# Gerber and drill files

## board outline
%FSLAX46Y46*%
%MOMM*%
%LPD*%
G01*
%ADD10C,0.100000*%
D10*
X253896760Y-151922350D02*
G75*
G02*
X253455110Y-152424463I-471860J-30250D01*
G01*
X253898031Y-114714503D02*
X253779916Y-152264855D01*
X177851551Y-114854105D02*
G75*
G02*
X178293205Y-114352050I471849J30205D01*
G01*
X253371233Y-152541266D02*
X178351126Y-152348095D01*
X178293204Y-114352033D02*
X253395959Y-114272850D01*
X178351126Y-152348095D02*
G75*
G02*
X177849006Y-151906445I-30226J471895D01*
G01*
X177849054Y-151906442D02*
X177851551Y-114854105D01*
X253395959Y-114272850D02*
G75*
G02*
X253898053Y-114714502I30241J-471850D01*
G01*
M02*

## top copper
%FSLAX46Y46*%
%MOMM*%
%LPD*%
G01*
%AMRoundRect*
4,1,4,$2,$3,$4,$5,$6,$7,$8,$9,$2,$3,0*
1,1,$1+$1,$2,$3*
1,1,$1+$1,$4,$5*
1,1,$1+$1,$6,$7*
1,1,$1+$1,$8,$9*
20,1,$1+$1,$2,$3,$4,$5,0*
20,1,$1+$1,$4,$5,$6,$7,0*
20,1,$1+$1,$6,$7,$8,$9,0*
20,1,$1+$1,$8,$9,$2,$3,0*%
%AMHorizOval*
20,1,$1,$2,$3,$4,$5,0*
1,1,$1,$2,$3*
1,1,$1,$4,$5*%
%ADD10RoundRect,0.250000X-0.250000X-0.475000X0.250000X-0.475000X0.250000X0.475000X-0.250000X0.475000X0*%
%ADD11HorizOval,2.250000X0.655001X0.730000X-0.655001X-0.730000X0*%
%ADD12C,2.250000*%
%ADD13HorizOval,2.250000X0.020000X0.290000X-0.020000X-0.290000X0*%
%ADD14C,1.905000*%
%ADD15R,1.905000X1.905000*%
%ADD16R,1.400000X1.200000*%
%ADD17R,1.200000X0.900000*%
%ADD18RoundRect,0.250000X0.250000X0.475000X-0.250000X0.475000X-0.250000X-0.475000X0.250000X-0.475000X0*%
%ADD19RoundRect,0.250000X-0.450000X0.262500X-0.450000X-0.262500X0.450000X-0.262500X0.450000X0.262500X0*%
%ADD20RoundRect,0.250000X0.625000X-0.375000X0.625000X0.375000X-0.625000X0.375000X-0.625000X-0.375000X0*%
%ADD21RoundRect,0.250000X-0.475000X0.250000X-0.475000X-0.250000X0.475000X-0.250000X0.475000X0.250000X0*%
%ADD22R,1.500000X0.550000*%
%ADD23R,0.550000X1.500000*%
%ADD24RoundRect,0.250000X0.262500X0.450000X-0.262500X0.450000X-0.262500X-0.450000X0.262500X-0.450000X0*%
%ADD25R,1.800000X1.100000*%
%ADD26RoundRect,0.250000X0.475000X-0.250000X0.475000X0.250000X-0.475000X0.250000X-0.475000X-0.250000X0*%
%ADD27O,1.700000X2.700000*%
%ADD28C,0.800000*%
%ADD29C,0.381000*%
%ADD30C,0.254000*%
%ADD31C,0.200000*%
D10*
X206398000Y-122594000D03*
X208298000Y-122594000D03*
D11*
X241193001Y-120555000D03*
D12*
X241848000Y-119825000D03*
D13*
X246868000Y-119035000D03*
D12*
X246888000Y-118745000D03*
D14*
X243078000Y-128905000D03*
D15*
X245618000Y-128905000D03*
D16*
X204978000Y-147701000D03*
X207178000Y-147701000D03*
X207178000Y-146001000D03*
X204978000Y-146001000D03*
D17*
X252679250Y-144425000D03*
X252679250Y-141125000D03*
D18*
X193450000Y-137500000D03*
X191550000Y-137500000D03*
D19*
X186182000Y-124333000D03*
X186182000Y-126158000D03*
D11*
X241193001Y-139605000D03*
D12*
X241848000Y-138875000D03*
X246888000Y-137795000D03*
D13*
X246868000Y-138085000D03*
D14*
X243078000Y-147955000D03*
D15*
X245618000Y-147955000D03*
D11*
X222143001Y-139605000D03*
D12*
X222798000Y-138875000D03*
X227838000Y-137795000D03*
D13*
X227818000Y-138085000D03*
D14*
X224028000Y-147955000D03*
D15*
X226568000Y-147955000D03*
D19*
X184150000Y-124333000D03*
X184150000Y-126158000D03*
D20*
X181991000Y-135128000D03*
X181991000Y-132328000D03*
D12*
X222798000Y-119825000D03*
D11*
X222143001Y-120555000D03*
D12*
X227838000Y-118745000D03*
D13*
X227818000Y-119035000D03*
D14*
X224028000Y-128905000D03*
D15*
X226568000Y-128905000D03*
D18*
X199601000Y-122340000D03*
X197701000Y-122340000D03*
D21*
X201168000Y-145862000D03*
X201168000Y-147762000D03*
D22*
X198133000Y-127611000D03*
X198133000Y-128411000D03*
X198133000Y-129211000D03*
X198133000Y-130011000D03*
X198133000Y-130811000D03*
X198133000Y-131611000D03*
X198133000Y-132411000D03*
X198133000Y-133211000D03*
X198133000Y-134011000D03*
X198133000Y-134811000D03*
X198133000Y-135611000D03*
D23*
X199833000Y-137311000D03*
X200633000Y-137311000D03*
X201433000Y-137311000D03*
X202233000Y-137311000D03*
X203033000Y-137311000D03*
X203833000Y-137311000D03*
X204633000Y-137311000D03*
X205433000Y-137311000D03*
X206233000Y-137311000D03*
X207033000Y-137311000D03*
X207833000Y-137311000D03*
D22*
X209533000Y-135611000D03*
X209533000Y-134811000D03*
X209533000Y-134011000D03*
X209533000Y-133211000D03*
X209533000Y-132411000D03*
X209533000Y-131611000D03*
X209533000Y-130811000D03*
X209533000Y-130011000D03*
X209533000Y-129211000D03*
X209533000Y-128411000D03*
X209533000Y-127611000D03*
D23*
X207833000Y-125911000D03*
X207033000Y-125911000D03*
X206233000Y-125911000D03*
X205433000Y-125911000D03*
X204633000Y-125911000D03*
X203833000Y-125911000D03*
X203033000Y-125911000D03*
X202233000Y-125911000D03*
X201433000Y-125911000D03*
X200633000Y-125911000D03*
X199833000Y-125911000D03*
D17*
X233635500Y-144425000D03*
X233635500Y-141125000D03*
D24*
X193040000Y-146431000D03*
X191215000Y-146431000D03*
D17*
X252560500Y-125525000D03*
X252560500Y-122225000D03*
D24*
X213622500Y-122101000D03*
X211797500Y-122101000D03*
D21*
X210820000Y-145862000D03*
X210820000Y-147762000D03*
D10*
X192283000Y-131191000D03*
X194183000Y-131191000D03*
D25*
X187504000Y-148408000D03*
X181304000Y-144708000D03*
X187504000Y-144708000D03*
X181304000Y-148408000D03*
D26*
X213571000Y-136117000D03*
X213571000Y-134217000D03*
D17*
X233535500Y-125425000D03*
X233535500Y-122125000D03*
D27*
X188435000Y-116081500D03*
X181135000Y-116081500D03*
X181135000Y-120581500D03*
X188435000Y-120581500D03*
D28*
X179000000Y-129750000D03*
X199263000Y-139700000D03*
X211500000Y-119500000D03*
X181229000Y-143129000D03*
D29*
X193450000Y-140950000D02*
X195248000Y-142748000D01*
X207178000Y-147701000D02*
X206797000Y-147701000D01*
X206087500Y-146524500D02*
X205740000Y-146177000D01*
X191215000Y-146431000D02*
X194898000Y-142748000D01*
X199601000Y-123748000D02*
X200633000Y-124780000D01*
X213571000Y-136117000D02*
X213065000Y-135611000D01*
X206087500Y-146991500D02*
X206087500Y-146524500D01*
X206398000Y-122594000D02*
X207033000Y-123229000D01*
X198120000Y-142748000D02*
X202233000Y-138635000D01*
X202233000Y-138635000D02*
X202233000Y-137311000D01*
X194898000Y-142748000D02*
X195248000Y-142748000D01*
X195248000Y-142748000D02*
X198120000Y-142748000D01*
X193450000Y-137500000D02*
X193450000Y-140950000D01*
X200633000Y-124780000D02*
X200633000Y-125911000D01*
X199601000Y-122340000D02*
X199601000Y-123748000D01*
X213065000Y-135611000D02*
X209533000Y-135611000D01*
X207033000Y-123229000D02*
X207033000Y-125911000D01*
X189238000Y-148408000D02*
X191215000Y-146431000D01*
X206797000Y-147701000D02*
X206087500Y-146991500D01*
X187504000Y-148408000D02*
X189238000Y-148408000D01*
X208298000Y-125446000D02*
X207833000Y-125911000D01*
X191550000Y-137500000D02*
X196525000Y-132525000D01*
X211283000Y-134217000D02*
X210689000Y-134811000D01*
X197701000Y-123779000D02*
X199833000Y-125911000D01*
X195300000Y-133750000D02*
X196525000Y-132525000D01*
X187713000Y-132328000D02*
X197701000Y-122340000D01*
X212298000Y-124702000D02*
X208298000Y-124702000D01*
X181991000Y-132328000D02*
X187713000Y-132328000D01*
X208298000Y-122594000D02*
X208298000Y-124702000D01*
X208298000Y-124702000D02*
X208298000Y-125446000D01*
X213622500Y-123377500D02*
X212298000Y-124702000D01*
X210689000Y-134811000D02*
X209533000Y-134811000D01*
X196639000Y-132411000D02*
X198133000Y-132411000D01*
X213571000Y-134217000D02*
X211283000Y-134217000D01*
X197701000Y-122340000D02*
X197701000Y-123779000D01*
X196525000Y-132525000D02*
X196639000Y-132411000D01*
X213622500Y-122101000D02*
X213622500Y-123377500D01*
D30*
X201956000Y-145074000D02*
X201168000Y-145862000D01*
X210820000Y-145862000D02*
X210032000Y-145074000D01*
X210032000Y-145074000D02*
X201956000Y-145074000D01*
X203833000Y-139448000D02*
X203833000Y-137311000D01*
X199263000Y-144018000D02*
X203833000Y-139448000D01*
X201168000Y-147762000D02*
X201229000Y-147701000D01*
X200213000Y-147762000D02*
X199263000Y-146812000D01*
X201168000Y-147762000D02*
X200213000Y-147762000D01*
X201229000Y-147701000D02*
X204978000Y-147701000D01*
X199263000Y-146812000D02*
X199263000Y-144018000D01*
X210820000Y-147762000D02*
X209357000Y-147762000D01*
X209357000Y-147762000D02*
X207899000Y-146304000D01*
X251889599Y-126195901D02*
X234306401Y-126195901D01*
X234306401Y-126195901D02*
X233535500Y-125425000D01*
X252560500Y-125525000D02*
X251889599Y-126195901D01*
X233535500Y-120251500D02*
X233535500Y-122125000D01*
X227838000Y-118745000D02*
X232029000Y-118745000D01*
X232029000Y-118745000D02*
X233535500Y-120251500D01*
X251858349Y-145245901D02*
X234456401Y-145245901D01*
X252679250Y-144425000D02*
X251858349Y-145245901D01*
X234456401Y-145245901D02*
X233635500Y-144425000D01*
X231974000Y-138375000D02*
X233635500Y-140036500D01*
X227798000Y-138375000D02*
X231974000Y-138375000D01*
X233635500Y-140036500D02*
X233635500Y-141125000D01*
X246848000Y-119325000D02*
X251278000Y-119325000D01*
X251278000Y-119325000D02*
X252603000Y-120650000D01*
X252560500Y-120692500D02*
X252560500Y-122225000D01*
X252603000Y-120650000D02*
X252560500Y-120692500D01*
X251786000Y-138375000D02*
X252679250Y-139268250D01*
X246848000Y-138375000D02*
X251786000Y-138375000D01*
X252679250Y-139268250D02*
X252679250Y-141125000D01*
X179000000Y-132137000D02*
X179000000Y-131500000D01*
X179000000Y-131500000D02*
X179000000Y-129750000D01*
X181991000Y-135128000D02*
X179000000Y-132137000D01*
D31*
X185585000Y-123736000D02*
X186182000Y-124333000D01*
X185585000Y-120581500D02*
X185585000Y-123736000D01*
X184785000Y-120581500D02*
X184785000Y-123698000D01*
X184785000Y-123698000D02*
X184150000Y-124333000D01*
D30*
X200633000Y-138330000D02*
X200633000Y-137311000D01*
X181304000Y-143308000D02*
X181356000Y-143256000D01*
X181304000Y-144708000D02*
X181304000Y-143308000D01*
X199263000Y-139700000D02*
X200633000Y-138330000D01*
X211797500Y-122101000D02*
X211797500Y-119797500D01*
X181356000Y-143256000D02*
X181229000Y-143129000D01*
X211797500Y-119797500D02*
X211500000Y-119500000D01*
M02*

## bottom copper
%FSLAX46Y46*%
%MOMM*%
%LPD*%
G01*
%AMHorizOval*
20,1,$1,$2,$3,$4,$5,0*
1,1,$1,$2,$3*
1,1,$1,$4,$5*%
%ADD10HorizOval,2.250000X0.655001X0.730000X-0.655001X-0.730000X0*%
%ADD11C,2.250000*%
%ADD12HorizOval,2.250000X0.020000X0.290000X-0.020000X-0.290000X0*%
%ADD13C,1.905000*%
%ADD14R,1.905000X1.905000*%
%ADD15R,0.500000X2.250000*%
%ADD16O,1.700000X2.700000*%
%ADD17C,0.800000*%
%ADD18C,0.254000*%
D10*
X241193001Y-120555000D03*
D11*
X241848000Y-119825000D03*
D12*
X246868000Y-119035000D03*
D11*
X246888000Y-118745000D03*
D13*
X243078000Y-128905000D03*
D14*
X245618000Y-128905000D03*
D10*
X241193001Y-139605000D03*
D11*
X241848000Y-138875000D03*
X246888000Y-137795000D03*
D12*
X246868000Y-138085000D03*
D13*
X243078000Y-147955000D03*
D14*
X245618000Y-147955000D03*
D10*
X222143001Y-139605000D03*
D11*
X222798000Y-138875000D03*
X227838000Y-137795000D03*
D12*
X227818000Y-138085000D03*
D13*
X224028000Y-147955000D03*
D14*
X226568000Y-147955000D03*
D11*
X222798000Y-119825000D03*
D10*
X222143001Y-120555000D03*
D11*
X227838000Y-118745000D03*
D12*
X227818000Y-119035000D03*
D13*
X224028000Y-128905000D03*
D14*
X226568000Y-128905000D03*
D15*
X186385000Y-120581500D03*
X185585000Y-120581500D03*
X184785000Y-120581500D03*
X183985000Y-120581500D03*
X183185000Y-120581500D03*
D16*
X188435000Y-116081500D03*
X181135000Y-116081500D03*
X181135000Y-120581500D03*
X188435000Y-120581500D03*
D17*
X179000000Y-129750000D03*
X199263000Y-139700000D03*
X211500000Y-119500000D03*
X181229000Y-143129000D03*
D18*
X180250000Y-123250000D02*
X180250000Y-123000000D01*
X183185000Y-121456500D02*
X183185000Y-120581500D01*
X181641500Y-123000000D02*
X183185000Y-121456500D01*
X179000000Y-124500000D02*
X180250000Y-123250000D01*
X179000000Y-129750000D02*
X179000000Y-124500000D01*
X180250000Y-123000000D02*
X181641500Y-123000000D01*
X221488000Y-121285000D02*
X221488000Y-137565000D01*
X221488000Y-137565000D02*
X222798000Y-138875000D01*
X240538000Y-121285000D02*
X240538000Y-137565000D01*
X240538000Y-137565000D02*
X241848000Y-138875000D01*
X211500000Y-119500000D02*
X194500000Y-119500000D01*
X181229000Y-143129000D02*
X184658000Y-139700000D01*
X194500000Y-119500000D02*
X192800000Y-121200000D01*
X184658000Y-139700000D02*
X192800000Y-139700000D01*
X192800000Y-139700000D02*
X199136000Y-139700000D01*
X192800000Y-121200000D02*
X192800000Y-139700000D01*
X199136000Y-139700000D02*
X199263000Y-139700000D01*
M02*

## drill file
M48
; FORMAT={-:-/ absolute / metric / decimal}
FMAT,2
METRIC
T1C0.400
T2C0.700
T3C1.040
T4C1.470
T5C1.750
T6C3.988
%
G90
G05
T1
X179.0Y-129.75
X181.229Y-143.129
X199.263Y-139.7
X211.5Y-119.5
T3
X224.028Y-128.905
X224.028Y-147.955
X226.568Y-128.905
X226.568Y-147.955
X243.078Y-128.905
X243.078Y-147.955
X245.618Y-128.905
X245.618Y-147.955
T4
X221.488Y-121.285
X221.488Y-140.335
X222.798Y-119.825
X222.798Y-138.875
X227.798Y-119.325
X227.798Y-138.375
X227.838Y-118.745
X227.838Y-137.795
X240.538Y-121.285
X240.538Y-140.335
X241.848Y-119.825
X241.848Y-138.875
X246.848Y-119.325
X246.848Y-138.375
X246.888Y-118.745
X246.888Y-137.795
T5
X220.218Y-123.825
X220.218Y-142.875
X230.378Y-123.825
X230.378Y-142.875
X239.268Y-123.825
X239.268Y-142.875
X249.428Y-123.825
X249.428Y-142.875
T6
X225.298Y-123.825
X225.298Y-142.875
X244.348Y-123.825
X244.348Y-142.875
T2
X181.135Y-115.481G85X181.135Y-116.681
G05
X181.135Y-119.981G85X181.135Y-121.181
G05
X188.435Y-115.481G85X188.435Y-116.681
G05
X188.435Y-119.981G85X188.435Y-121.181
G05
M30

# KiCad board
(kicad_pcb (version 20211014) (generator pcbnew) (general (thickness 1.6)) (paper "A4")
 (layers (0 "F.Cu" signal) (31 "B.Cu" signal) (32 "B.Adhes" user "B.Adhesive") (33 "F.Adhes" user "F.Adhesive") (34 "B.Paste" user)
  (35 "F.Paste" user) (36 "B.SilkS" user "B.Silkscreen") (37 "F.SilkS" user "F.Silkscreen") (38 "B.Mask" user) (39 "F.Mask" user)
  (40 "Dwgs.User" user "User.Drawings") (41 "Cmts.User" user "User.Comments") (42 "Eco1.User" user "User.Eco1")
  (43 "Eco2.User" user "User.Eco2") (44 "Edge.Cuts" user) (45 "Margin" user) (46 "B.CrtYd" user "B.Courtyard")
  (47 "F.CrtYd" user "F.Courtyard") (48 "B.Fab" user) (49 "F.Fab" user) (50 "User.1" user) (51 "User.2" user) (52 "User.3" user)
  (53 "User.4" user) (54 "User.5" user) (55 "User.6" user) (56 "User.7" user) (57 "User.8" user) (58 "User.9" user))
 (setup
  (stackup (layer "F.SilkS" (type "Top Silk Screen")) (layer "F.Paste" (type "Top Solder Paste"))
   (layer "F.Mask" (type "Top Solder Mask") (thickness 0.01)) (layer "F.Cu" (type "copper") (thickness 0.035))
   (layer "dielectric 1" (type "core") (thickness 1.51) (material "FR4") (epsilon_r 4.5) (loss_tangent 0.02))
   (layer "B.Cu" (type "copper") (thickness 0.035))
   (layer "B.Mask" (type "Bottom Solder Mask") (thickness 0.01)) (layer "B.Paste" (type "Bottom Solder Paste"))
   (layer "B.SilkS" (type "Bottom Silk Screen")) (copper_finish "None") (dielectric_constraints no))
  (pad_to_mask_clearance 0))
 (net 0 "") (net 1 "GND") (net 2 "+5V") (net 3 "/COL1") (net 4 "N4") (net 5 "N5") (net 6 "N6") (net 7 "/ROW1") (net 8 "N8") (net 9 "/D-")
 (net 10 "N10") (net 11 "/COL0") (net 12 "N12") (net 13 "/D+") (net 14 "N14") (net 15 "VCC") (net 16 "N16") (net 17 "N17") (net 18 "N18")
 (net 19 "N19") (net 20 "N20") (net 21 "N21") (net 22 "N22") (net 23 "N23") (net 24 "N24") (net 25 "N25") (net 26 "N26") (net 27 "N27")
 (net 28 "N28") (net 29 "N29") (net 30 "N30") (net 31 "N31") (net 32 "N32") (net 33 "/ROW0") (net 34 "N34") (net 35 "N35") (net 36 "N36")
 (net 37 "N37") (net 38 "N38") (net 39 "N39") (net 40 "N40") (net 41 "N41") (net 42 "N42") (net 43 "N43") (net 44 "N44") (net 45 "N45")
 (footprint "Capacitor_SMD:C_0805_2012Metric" (layer "F.Cu") (at 207.348 122.594)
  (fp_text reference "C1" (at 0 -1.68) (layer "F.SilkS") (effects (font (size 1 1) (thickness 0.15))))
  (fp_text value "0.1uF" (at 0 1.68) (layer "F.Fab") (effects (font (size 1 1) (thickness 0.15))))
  (pad "1" smd roundrect (at -0.95 0) (size 1 1.45) (layers "F.Cu" "F.Paste" "F.Mask") (roundrect_rratio 0.25) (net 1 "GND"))
  (pad "2" smd roundrect (at 0.95 0) (size 1 1.45) (layers "F.Cu" "F.Paste" "F.Mask") (roundrect_rratio 0.25) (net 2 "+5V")))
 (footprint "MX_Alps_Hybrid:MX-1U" (layer "F.Cu") (at 244.348 123.825)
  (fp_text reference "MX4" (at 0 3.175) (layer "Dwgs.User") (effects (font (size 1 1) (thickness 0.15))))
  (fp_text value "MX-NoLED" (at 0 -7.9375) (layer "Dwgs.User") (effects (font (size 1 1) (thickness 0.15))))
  (pad "" np_thru_hole circle locked (at 0 0) (size 3.9878 3.9878) (drill 3.9878) (layers *.Cu *.Mask))
  (pad "" np_thru_hole circle locked (at 5.08 0 48.0996) (size 1.75 1.75) (drill 1.75) (layers *.Cu *.Mask))
  (pad "" np_thru_hole circle locked (at -5.08 0 48.0996) (size 1.75 1.75) (drill 1.75) (layers *.Cu *.Mask))
  (pad "1" thru_hole oval locked (at -3.81 -2.54 48.0996) (size 4.211556 2.25) (drill 1.47 (offset 0.980778 0)) (layers *.Cu "B.Mask")
   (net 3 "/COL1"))
  (pad "1" thru_hole circle locked (at -2.5 -4) (size 2.25 2.25) (drill 1.47) (layers *.Cu "B.Mask") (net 3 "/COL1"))
  (pad "2" thru_hole oval locked (at 2.5 -4.5 86.0548) (size 2.831378 2.25) (drill 1.47 (offset 0.290689 0)) (layers *.Cu "B.Mask")
   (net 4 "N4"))
  (pad "2" thru_hole circle locked (at 2.54 -5.08) (size 2.25 2.25) (drill 1.47) (layers *.Cu "B.Mask") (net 4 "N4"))
  (pad "3" thru_hole circle locked (at -1.27 5.08) (size 1.905 1.905) (drill 1.04) (layers *.Cu "B.Mask"))
  (pad "4" thru_hole rect locked (at 1.27 5.08) (size 1.905 1.905) (drill 1.04) (layers *.Cu "B.Mask")))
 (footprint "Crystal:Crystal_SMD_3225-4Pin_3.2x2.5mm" (layer "F.Cu") (at 206.078 146.851)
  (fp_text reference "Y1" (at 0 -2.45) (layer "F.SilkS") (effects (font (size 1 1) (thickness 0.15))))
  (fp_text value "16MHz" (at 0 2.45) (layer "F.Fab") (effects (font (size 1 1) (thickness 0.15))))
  (pad "1" smd rect (at -1.1 0.85) (size 1.4 1.2) (layers "F.Cu" "F.Paste" "F.Mask") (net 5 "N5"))
  (pad "2" smd rect (at 1.1 0.85) (size 1.4 1.2) (layers "F.Cu" "F.Paste" "F.Mask") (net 1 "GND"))
  (pad "3" smd rect (at 1.1 -0.85) (size 1.4 1.2) (layers "F.Cu" "F.Paste" "F.Mask") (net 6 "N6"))
  (pad "4" smd rect (at -1.1 -0.85) (size 1.4 1.2) (layers "F.Cu" "F.Paste" "F.Mask") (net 1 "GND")))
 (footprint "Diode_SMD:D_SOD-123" (layer "F.Cu") (at 252.67925 142.775 90)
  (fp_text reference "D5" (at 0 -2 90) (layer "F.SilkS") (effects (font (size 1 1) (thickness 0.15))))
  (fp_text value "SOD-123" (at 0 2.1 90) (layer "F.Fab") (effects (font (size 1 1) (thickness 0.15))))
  (pad "1" smd rect (at -1.65 0 90) (size 0.9 1.2) (layers "F.Cu" "F.Paste" "F.Mask") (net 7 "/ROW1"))
  (pad "2" smd rect (at 1.65 0 90) (size 0.9 1.2) (layers "F.Cu" "F.Paste" "F.Mask") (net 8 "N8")))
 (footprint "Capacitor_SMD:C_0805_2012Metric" (layer "F.Cu") (at 192.5 137.5 180)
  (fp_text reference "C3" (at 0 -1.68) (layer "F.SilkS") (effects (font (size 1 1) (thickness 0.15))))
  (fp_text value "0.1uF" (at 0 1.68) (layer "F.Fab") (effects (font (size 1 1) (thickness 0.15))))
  (pad "1" smd roundrect (at -0.95 0 180) (size 1 1.45) (layers "F.Cu" "F.Paste" "F.Mask") (roundrect_rratio 0.25) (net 1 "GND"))
  (pad "2" smd roundrect (at 0.95 0 180) (size 1 1.45) (layers "F.Cu" "F.Paste" "F.Mask") (roundrect_rratio 0.25) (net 2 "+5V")))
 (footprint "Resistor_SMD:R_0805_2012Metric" (layer "F.Cu") (at 186.182 125.2455 -90)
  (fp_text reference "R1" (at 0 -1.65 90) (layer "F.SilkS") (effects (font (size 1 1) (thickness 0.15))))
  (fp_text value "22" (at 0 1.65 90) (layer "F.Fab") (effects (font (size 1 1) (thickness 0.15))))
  (pad "1" smd roundrect (at -0.9125 0 270) (size 1.025 1.4) (layers "F.Cu" "F.Paste" "F.Mask") (roundrect_rratio 0.243902) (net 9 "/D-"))
  (pad "2" smd roundrect (at 0.9125 0 270) (size 1.025 1.4) (layers "F.Cu" "F.Paste" "F.Mask") (roundrect_rratio 0.243902) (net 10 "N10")))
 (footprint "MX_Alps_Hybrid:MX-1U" (layer "F.Cu") (at 244.348 142.875)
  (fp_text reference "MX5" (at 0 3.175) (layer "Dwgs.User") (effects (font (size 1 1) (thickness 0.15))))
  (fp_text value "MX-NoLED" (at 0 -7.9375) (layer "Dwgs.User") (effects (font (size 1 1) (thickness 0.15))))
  (pad "" np_thru_hole circle locked (at 5.08 0 48.0996) (size 1.75 1.75) (drill 1.75) (layers *.Cu *.Mask))
  (pad "" np_thru_hole circle locked (at 0 0) (size 3.9878 3.9878) (drill 3.9878) (layers *.Cu *.Mask))
  (pad "" np_thru_hole circle locked (at -5.08 0 48.0996) (size 1.75 1.75) (drill 1.75) (layers *.Cu *.Mask))
  (pad "1" thru_hole oval locked (at -3.81 -2.54 48.0996) (size 4.211556 2.25) (drill 1.47 (offset 0.980778 0)) (layers *.Cu "B.Mask")
   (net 3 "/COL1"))
  (pad "1" thru_hole circle locked (at -2.5 -4) (size 2.25 2.25) (drill 1.47) (layers *.Cu "B.Mask") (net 3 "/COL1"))
  (pad "2" thru_hole circle locked (at 2.54 -5.08) (size 2.25 2.25) (drill 1.47) (layers *.Cu "B.Mask") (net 8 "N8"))
  (pad "2" thru_hole oval locked (at 2.5 -4.5 86.0548) (size 2.831378 2.25) (drill 1.47 (offset 0.290689 0)) (layers *.Cu "B.Mask")
   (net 8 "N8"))
  (pad "3" thru_hole circle locked (at -1.27 5.08) (size 1.905 1.905) (drill 1.04) (layers *.Cu "B.Mask"))
  (pad "4" thru_hole rect locked (at 1.27 5.08) (size 1.905 1.905) (drill 1.04) (layers *.Cu "B.Mask")))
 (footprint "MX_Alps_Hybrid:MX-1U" (layer "F.Cu") (at 225.298 142.875)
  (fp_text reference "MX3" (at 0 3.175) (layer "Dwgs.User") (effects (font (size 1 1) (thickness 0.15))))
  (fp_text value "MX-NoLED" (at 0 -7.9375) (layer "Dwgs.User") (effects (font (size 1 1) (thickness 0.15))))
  (pad "" np_thru_hole circle locked (at 5.08 0 48.0996) (size 1.75 1.75) (drill 1.75) (layers *.Cu *.Mask))
  (pad "" np_thru_hole circle locked (at 0 0) (size 3.9878 3.9878) (drill 3.9878) (layers *.Cu *.Mask))
  (pad "" np_thru_hole circle locked (at -5.08 0 48.0996) (size 1.75 1.75) (drill 1.75) (layers *.Cu *.Mask))
  (pad "1" thru_hole oval locked (at -3.81 -2.54 48.0996) (size 4.211556 2.25) (drill 1.47 (offset 0.980778 0)) (layers *.Cu "B.Mask")
   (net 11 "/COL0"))
  (pad "1" thru_hole circle locked (at -2.5 -4) (size 2.25 2.25) (drill 1.47) (layers *.Cu "B.Mask") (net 11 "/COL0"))
  (pad "2" thru_hole circle locked (at 2.54 -5.08) (size 2.25 2.25) (drill 1.47) (layers *.Cu "B.Mask") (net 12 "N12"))
  (pad "2" thru_hole oval locked (at 2.5 -4.5 86.0548) (size 2.831378 2.25) (drill 1.47 (offset 0.290689 0)) (layers *.Cu "B.Mask")
   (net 12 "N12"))
  (pad "3" thru_hole circle locked (at -1.27 5.08) (size 1.905 1.905) (drill 1.04) (layers *.Cu "B.Mask"))
  (pad "4" thru_hole rect locked (at 1.27 5.08) (size 1.905 1.905) (drill 1.04) (layers *.Cu "B.Mask")))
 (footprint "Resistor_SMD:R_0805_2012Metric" (layer "F.Cu") (at 184.15 125.2455 -90)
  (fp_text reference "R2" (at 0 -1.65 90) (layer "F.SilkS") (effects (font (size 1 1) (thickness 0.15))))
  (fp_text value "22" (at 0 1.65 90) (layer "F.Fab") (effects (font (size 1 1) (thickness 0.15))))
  (pad "1" smd roundrect (at -0.9125 0 270) (size 1.025 1.4) (layers "F.Cu" "F.Paste" "F.Mask") (roundrect_rratio 0.243902) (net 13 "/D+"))
  (pad "2" smd roundrect (at 0.9125 0 270) (size 1.025 1.4) (layers "F.Cu" "F.Paste" "F.Mask") (roundrect_rratio 0.243902) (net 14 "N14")))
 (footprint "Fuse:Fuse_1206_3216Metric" (layer "F.Cu") (at 181.991 133.728 90)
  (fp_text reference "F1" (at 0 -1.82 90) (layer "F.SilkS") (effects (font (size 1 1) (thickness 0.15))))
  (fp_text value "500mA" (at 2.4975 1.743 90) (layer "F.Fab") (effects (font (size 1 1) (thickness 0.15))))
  (pad "1" smd roundrect (at -1.4 0 90) (size 1.25 1.75) (layers "F.Cu" "F.Paste" "F.Mask") (roundrect_rratio 0.2) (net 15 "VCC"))
  (pad "2" smd roundrect (at 1.4 0 90) (size 1.25 1.75) (layers "F.Cu" "F.Paste" "F.Mask") (roundrect_rratio 0.2) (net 2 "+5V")))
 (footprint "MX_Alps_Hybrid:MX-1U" (layer "F.Cu") (at 225.298 123.825)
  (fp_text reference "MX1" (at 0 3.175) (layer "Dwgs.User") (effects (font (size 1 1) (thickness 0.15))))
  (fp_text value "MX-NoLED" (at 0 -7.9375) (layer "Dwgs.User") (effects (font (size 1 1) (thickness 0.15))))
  (pad "" np_thru_hole circle locked (at -5.08 0 48.0996) (size 1.75 1.75) (drill 1.75) (layers *.Cu *.Mask))
  (pad "" np_thru_hole circle locked (at 5.08 0 48.0996) (size 1.75 1.75) (drill 1.75) (layers *.Cu *.Mask))
  (pad "" np_thru_hole circle locked (at 0 0) (size 3.9878 3.9878) (drill 3.9878) (layers *.Cu *.Mask))
  (pad "1" thru_hole circle locked (at -2.5 -4) (size 2.25 2.25) (drill 1.47) (layers *.Cu "B.Mask") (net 11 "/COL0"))
  (pad "1" thru_hole oval locked (at -3.81 -2.54 48.0996) (size 4.211556 2.25) (drill 1.47 (offset 0.980778 0)) (layers *.Cu "B.Mask")
   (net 11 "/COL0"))
  (pad "2" thru_hole circle locked (at 2.54 -5.08) (size 2.25 2.25) (drill 1.47) (layers *.Cu "B.Mask") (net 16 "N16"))
  (pad "2" thru_hole oval locked (at 2.5 -4.5 86.0548) (size 2.831378 2.25) (drill 1.47 (offset 0.290689 0)) (layers *.Cu "B.Mask")
   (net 16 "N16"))
  (pad "3" thru_hole circle locked (at -1.27 5.08) (size 1.905 1.905) (drill 1.04) (layers *.Cu "B.Mask"))
  (pad "4" thru_hole rect locked (at 1.27 5.08) (size 1.905 1.905) (drill 1.04) (layers *.Cu "B.Mask")))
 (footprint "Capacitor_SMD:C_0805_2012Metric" (layer "F.Cu") (at 198.651 122.34 180)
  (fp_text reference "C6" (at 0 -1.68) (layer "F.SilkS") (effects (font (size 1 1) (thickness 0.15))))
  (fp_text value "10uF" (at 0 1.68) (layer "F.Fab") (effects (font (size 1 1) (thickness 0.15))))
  (pad "1" smd roundrect (at -0.95 0 180) (size 1 1.45) (layers "F.Cu" "F.Paste" "F.Mask") (roundrect_rratio 0.25) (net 1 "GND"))
  (pad "2" smd roundrect (at 0.95 0 180) (size 1 1.45) (layers "F.Cu" "F.Paste" "F.Mask") (roundrect_rratio 0.25) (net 2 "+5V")))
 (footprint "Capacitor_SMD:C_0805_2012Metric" (layer "F.Cu") (at 201.168 146.812 -90)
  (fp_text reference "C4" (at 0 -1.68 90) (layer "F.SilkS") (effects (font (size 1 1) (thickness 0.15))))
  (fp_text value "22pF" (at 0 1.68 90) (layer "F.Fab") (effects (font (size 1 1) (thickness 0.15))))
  (pad "1" smd roundrect (at -0.95 0 270) (size 1 1.45) (layers "F.Cu" "F.Paste" "F.Mask") (roundrect_rratio 0.25) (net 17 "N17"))
  (pad "2" smd roundrect (at 0.95 0 270) (size 1 1.45) (layers "F.Cu" "F.Paste" "F.Mask") (roundrect_rratio 0.25) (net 5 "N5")))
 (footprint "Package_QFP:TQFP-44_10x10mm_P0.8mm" (layer "F.Cu") (at 203.833 131.611)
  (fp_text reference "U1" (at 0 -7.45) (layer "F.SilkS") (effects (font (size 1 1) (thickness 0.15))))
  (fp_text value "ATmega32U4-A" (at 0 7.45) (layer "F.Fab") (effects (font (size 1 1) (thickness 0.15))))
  (pad "1" smd rect (at -5.7 -4) (size 1.5 0.55) (layers "F.Cu" "F.Paste" "F.Mask") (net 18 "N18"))
  (pad "2" smd rect (at -5.7 -3.2) (size 1.5 0.55) (layers "F.Cu" "F.Paste" "F.Mask") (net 2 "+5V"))
  (pad "3" smd rect (at -5.7 -2.4) (size 1.5 0.55) (layers "F.Cu" "F.Paste" "F.Mask") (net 10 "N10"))
  (pad "4" smd rect (at -5.7 -1.6) (size 1.5 0.55) (layers "F.Cu" "F.Paste" "F.Mask") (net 14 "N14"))
  (pad "5" smd rect (at -5.7 -0.8) (size 1.5 0.55) (layers "F.Cu" "F.Paste" "F.Mask") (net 1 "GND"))
  (pad "6" smd rect (at -5.7 0) (size 1.5 0.55) (layers "F.Cu" "F.Paste" "F.Mask") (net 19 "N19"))
  (pad "7" smd rect (at -5.7 0.8) (size 1.5 0.55) (layers "F.Cu" "F.Paste" "F.Mask") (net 2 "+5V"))
  (pad "8" smd rect (at -5.7 1.6) (size 1.5 0.55) (layers "F.Cu" "F.Paste" "F.Mask") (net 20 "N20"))
  (pad "9" smd rect (at -5.7 2.4) (size 1.5 0.55) (layers "F.Cu" "F.Paste" "F.Mask") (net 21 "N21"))
  (pad "10" smd rect (at -5.7 3.2) (size 1.5 0.55) (layers "F.Cu" "F.Paste" "F.Mask") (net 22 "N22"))
  (pad "11" smd rect (at -5.7 4) (size 1.5 0.55) (layers "F.Cu" "F.Paste" "F.Mask") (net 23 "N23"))
  (pad "12" smd rect (at -4 5.7 90) (size 1.5 0.55) (layers "F.Cu" "F.Paste" "F.Mask") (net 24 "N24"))
  (pad "13" smd rect (at -3.2 5.7 90) (size 1.5 0.55) (layers "F.Cu" "F.Paste" "F.Mask") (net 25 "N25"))
  (pad "14" smd rect (at -2.4 5.7 90) (size 1.5 0.55) (layers "F.Cu" "F.Paste" "F.Mask") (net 2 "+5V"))
  (pad "15" smd rect (at -1.6 5.7 90) (size 1.5 0.55) (layers "F.Cu" "F.Paste" "F.Mask") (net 1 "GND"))
  (pad "16" smd rect (at -0.8 5.7 90) (size 1.5 0.55) (layers "F.Cu" "F.Paste" "F.Mask") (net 6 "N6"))
  (pad "17" smd rect (at 0 5.7 90) (size 1.5 0.55) (layers "F.Cu" "F.Paste" "F.Mask") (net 5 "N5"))
  (pad "18" smd rect (at 0.8 5.7 90) (size 1.5 0.55) (layers "F.Cu" "F.Paste" "F.Mask") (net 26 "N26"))
  (pad "19" smd rect (at 1.6 5.7 90) (size 1.5 0.55) (layers "F.Cu" "F.Paste" "F.Mask") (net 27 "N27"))
  (pad "20" smd rect (at 2.4 5.7 90) (size 1.5 0.55) (layers "F.Cu" "F.Paste" "F.Mask") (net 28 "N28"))
  (pad "21" smd rect (at 3.2 5.7 90) (size 1.5 0.55) (layers "F.Cu" "F.Paste" "F.Mask") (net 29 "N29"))
  (pad "22" smd rect (at 4 5.7 90) (size 1.5 0.55) (layers "F.Cu" "F.Paste" "F.Mask") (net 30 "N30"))
  (pad "23" smd rect (at 5.7 4) (size 1.5 0.55) (layers "F.Cu" "F.Paste" "F.Mask") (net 1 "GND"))
  (pad "24" smd rect (at 5.7 3.2) (size 1.5 0.55) (layers "F.Cu" "F.Paste" "F.Mask") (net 2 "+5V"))
  (pad "25" smd rect (at 5.7 2.4) (size 1.5 0.55) (layers "F.Cu" "F.Paste" "F.Mask") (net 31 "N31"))
  (pad "26" smd rect (at 5.7 1.6) (size 1.5 0.55) (layers "F.Cu" "F.Paste" "F.Mask") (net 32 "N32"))
  (pad "27" smd rect (at 5.7 0.8) (size 1.5 0.55) (layers "F.Cu" "F.Paste" "F.Mask") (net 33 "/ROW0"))
  (pad "28" smd rect (at 5.7 0) (size 1.5 0.55) (layers "F.Cu" "F.Paste" "F.Mask") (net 3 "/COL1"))
  (pad "29" smd rect (at 5.7 -0.8) (size 1.5 0.55) (layers "F.Cu" "F.Paste" "F.Mask") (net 11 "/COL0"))
  (pad "30" smd rect (at 5.7 -1.6) (size 1.5 0.55) (layers "F.Cu" "F.Paste" "F.Mask") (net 7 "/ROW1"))
  (pad "31" smd rect (at 5.7 -2.4) (size 1.5 0.55) (layers "F.Cu" "F.Paste" "F.Mask") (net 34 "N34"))
  (pad "32" smd rect (at 5.7 -3.2) (size 1.5 0.55) (layers "F.Cu" "F.Paste" "F.Mask") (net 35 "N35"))
  (pad "33" smd rect (at 5.7 -4) (size 1.5 0.55) (layers "F.Cu" "F.Paste" "F.Mask") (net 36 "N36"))
  (pad "34" smd rect (at 4 -5.7 90) (size 1.5 0.55) (layers "F.Cu" "F.Paste" "F.Mask") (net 2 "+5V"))
  (pad "35" smd rect (at 3.2 -5.7 90) (size 1.5 0.55) (layers "F.Cu" "F.Paste" "F.Mask") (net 1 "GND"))
  (pad "36" smd rect (at 2.4 -5.7 90) (size 1.5 0.55) (layers "F.Cu" "F.Paste" "F.Mask") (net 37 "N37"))
  (pad "37" smd rect (at 1.6 -5.7 90) (size 1.5 0.55) (layers "F.Cu" "F.Paste" "F.Mask") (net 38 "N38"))
  (pad "38" smd rect (at 0.8 -5.7 90) (size 1.5 0.55) (layers "F.Cu" "F.Paste" "F.Mask") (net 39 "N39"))
  (pad "39" smd rect (at 0 -5.7 90) (size 1.5 0.55) (layers "F.Cu" "F.Paste" "F.Mask") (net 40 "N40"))
  (pad "40" smd rect (at -0.8 -5.7 90) (size 1.5 0.55) (layers "F.Cu" "F.Paste" "F.Mask") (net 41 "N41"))
  (pad "41" smd rect (at -1.6 -5.7 90) (size 1.5 0.55) (layers "F.Cu" "F.Paste" "F.Mask") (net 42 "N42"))
  (pad "42" smd rect (at -2.4 -5.7 90) (size 1.5 0.55) (layers "F.Cu" "F.Paste" "F.Mask") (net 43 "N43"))
  (pad "43" smd rect (at -3.2 -5.7 90) (size 1.5 0.55) (layers "F.Cu" "F.Paste" "F.Mask") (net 1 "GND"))
  (pad "44" smd rect (at -4 -5.7 90) (size 1.5 0.55) (layers "F.Cu" "F.Paste" "F.Mask") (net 2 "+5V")))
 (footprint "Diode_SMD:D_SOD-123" (layer "F.Cu") (at 233.6355 142.775 90)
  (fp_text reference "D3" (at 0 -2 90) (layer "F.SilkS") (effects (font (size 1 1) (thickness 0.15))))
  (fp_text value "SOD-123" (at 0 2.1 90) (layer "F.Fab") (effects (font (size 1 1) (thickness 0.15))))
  (pad "1" smd rect (at -1.65 0 90) (size 0.9 1.2) (layers "F.Cu" "F.Paste" "F.Mask") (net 7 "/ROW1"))
  (pad "2" smd rect (at 1.65 0 90) (size 0.9 1.2) (layers "F.Cu" "F.Paste" "F.Mask") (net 12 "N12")))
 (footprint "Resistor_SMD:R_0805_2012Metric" (layer "F.Cu") (at 192.1275 146.431 180)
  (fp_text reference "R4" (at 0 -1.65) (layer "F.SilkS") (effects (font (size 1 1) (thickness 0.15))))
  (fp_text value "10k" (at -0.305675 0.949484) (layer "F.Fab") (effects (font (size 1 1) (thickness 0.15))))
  (pad "1" smd roundrect (at -0.9125 0 180) (size 1.025 1.4) (layers "F.Cu" "F.Paste" "F.Mask") (roundrect_rratio 0.243902) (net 36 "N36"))
  (pad "2" smd roundrect (at 0.9125 0 180) (size 1.025 1.4) (layers "F.Cu" "F.Paste" "F.Mask") (roundrect_rratio 0.243902) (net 1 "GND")))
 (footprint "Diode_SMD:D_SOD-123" (layer "F.Cu") (at 252.5605 123.875 90)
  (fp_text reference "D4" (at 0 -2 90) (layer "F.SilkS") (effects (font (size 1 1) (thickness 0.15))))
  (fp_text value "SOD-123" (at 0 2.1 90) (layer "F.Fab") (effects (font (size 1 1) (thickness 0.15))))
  (pad "1" smd rect (at -1.65 0 90) (size 0.9 1.2) (layers "F.Cu" "F.Paste" "F.Mask") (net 33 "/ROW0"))
  (pad "2" smd rect (at 1.65 0 90) (size 0.9 1.2) (layers "F.Cu" "F.Paste" "F.Mask") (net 4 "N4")))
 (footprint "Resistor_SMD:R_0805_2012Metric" (layer "F.Cu") (at 212.71 122.101 180)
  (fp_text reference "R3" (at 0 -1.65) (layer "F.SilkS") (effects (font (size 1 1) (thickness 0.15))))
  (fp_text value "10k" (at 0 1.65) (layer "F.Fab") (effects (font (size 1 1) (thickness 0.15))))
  (pad "1" smd roundrect (at -0.9125 0 180) (size 1.025 1.4) (layers "F.Cu" "F.Paste" "F.Mask") (roundrect_rratio 0.243902) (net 2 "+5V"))
  (pad "2" smd roundrect (at 0.9125 0 180) (size 1.025 1.4) (layers "F.Cu" "F.Paste" "F.Mask") (roundrect_rratio 0.243902) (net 25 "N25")))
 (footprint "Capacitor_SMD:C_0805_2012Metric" (layer "F.Cu") (at 210.82 146.812 -90)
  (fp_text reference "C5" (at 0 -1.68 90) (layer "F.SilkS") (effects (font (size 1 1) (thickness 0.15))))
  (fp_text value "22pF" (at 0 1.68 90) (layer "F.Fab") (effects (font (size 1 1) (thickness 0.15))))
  (pad "1" smd roundrect (at -0.95 0 270) (size 1 1.45) (layers "F.Cu" "F.Paste" "F.Mask") (roundrect_rratio 0.25) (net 17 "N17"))
  (pad "2" smd roundrect (at 0.95 0 270) (size 1 1.45) (layers "F.Cu" "F.Paste" "F.Mask") (roundrect_rratio 0.25) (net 6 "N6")))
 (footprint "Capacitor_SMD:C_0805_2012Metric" (layer "F.Cu") (at 193.233 131.191)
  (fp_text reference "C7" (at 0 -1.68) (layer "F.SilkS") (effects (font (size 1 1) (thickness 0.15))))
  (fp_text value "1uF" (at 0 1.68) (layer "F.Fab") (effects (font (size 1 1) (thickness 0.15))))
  (pad "1" smd roundrect (at -0.95 0) (size 1 1.45) (layers "F.Cu" "F.Paste" "F.Mask") (roundrect_rratio 0.25) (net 1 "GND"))
  (pad "2" smd roundrect (at 0.95 0) (size 1 1.45) (layers "F.Cu" "F.Paste" "F.Mask") (roundrect_rratio 0.25) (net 19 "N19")))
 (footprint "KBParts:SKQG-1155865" (layer "F.Cu") (at 184.404 146.558)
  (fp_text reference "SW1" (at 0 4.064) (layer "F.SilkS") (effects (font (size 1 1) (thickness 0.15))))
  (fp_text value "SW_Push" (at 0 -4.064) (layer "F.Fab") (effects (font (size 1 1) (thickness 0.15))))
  (pad "1" smd rect locked (at 3.1 1.85) (size 1.8 1.1) (layers "F.Cu" "F.Paste" "F.Mask") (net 1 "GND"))
  (pad "2" smd rect locked (at -3.1 -1.85) (size 1.8 1.1) (layers "F.Cu" "F.Paste" "F.Mask") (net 25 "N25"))
  (pad "3" smd rect locked (at 3.1 -1.85) (size 1.8 1.1) (layers "F.Cu" "F.Paste" "F.Mask"))
  (pad "4" smd rect locked (at -3.1 1.85) (size 1.8 1.1) (layers "F.Cu" "F.Paste" "F.Mask")))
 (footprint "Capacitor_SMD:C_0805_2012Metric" (layer "F.Cu") (at 213.571 135.167 90)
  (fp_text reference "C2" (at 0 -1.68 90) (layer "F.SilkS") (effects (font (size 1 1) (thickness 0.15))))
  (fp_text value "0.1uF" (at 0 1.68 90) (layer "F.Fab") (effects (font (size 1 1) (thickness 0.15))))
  (pad "1" smd roundrect (at -0.95 0 90) (size 1 1.45) (layers "F.Cu" "F.Paste" "F.Mask") (roundrect_rratio 0.25) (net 1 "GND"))
  (pad "2" smd roundrect (at 0.95 0 90) (size 1 1.45) (layers "F.Cu" "F.Paste" "F.Mask") (roundrect_rratio 0.25) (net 2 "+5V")))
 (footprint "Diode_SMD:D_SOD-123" (layer "F.Cu") (at 233.5355 123.775 90)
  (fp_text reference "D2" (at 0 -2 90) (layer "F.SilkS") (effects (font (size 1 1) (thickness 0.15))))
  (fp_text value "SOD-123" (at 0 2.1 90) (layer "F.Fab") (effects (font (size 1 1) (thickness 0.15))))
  (pad "1" smd rect (at -1.65 0 90) (size 0.9 1.2) (layers "F.Cu" "F.Paste" "F.Mask") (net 33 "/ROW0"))
  (pad "2" smd rect (at 1.65 0 90) (size 0.9 1.2) (layers "F.Cu" "F.Paste" "F.Mask") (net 16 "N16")))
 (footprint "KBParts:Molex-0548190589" (layer "B.Cu") (at 184.785 116.0815 -90)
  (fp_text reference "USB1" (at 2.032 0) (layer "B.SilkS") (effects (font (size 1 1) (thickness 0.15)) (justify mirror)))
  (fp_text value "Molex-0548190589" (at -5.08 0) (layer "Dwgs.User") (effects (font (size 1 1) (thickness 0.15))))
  (pad "1" smd rect locked (at 4.5 -1.6 270) (size 2.25 0.5) (layers "B.Cu" "B.Paste" "B.Mask") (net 1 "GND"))
  (pad "2" smd rect locked (at 4.5 -0.8 270) (size 2.25 0.5) (layers "B.Cu" "B.Paste" "B.Mask") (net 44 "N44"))
  (pad "3" smd rect locked (at 4.5 0 270) (size 2.25 0.5) (layers "B.Cu" "B.Paste" "B.Mask") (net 13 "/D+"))
  (pad "4" smd rect locked (at 4.5 0.8 270) (size 2.25 0.5) (layers "B.Cu" "B.Paste" "B.Mask") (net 9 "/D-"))
  (pad "5" smd rect locked (at 4.5 1.6 270) (size 2.25 0.5) (layers "B.Cu" "B.Paste" "B.Mask") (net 15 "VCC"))
  (pad "6" thru_hole oval locked (at 0 -3.65 270) (size 2.7 1.7) (drill oval 1.9 0.7) (layers *.Cu *.Mask) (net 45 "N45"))
  (pad "6" thru_hole oval locked (at 0 3.65 270) (size 2.7 1.7) (drill oval 1.9 0.7) (layers *.Cu *.Mask) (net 45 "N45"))
  (pad "6" thru_hole oval locked (at 4.5 3.65 270) (size 2.7 1.7) (drill oval 1.9 0.7) (layers *.Cu *.Mask) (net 45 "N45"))
  (pad "6" thru_hole oval locked (at 4.5 -3.65 270) (size 2.7 1.7) (drill oval 1.9 0.7) (layers *.Cu *.Mask) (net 45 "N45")))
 (gr_arc (start 253.89676 151.92235) (mid 253.779916 152.264855) (end 253.455107 152.424422) (layer "Edge.Cuts") (width 0.1))
 (gr_line (start 253.898031 114.714503) (end 253.779916 152.264855) (layer "Edge.Cuts") (width 0.1))
 (gr_arc (start 177.851551 114.854105) (mid 177.968395 114.5116) (end 178.293204 114.352033) (layer "Edge.Cuts") (width 0.1))
 (gr_line (start 253.371233 152.541266) (end 178.351126 152.348095) (layer "Edge.Cuts") (width 0.1))
 (gr_line (start 178.293204 114.352033) (end 253.395959 114.27285) (layer "Edge.Cuts") (width 0.1))
 (gr_arc (start 178.351126 152.348095) (mid 178.008621 152.231251) (end 177.849054 151.906442) (layer "Edge.Cuts") (width 0.1))
 (gr_line (start 177.849054 151.906442) (end 177.851551 114.854105) (layer "Edge.Cuts") (width 0.1))
 (gr_arc (start 253.395959 114.27285) (mid 253.738465 114.389694) (end 253.898031 114.714503) (layer "Edge.Cuts") (width 0.1))
 (segment (start 193.45 140.95) (end 195.248 142.748) (width 0.381) (layer "F.Cu") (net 1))
 (segment (start 207.178 147.701) (end 206.797 147.701) (width 0.381) (layer "F.Cu") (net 1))
 (segment (start 206.0875 146.5245) (end 205.74 146.177) (width 0.381) (layer "F.Cu") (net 1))
 (segment (start 191.215 146.431) (end 194.898 142.748) (width 0.381) (layer "F.Cu") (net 1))
 (segment (start 199.601 123.748) (end 200.633 124.78) (width 0.381) (layer "F.Cu") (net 1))
 (segment (start 213.571 136.117) (end 213.065 135.611) (width 0.381) (layer "F.Cu") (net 1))
 (segment (start 206.0875 146.9915) (end 206.0875 146.5245) (width 0.381) (layer "F.Cu") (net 1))
 (segment (start 206.398 122.594) (end 207.033 123.229) (width 0.381) (layer "F.Cu") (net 1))
 (segment (start 198.12 142.748) (end 202.233 138.635) (width 0.381) (layer "F.Cu") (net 1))
 (segment (start 202.233 138.635) (end 202.233 137.311) (width 0.381) (layer "F.Cu") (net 1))
 (segment (start 194.898 142.748) (end 195.248 142.748) (width 0.381) (layer "F.Cu") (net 1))
 (segment (start 195.248 142.748) (end 198.12 142.748) (width 0.381) (layer "F.Cu") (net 1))
 (segment (start 193.45 137.5) (end 193.45 140.95) (width 0.381) (layer "F.Cu") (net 1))
 (segment (start 200.633 124.78) (end 200.633 125.911) (width 0.381) (layer "F.Cu") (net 1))
 (segment (start 199.601 122.34) (end 199.601 123.748) (width 0.381) (layer "F.Cu") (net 1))
 (segment (start 213.065 135.611) (end 209.533 135.611) (width 0.381) (layer "F.Cu") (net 1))
 (segment (start 207.033 123.229) (end 207.033 125.911) (width 0.381) (layer "F.Cu") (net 1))
 (segment (start 189.238 148.408) (end 191.215 146.431) (width 0.381) (layer "F.Cu") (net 1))
 (segment (start 206.797 147.701) (end 206.0875 146.9915) (width 0.381) (layer "F.Cu") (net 1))
 (segment (start 187.504 148.408) (end 189.238 148.408) (width 0.381) (layer "F.Cu") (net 1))
 (segment (start 208.298 125.446) (end 207.833 125.911) (width 0.381) (layer "F.Cu") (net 2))
 (segment (start 191.55 137.5) (end 196.525 132.525) (width 0.381) (layer "F.Cu") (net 2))
 (segment (start 211.283 134.217) (end 210.689 134.811) (width 0.381) (layer "F.Cu") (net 2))
 (segment (start 197.701 123.779) (end 199.833 125.911) (width 0.381) (layer "F.Cu") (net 2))
 (segment (start 195.3 133.75) (end 196.525 132.525) (width 0.381) (layer "F.Cu") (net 2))
 (segment (start 187.713 132.328) (end 197.701 122.34) (width 0.381) (layer "F.Cu") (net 2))
 (segment (start 212.298 124.702) (end 208.298 124.702) (width 0.381) (layer "F.Cu") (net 2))
 (segment (start 181.991 132.328) (end 187.713 132.328) (width 0.381) (layer "F.Cu") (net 2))
 (segment (start 208.298 122.594) (end 208.298 124.702) (width 0.381) (layer "F.Cu") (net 2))
 (segment (start 208.298 124.702) (end 208.298 125.446) (width 0.381) (layer "F.Cu") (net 2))
 (segment (start 213.6225 123.3775) (end 212.298 124.702) (width 0.381) (layer "F.Cu") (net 2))
 (segment (start 210.689 134.811) (end 209.533 134.811) (width 0.381) (layer "F.Cu") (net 2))
 (segment (start 196.639 132.411) (end 198.133 132.411) (width 0.381) (layer "F.Cu") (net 2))
 (segment (start 213.571 134.217) (end 211.283 134.217) (width 0.381) (layer "F.Cu") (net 2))
 (segment (start 197.701 122.34) (end 197.701 123.779) (width 0.381) (layer "F.Cu") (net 2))
 (segment (start 196.525 132.525) (end 196.639 132.411) (width 0.381) (layer "F.Cu") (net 2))
 (segment (start 213.6225 122.101) (end 213.6225 123.3775) (width 0.381) (layer "F.Cu") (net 2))
 (segment (start 201.956 145.074) (end 201.168 145.862) (width 0.254) (layer "F.Cu") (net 17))
 (segment (start 210.82 145.862) (end 210.032 145.074) (width 0.254) (layer "F.Cu") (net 17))
 (segment (start 210.032 145.074) (end 201.956 145.074) (width 0.254) (layer "F.Cu") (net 17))
 (segment (start 203.833 139.448) (end 203.833 137.311) (width 0.254) (layer "F.Cu") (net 5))
 (segment (start 199.263 144.018) (end 203.833 139.448) (width 0.254) (layer "F.Cu") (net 5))
 (segment (start 201.168 147.762) (end 201.229 147.701) (width 0.254) (layer "F.Cu") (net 5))
 (segment (start 200.213 147.762) (end 199.263 146.812) (width 0.254) (layer "F.Cu") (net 5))
 (segment (start 201.168 147.762) (end 200.213 147.762) (width 0.254) (layer "F.Cu") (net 5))
 (segment (start 201.229 147.701) (end 204.978 147.701) (width 0.254) (layer "F.Cu") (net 5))
 (segment (start 199.263 146.812) (end 199.263 144.018) (width 0.254) (layer "F.Cu") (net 5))
 (segment (start 210.82 147.762) (end 209.357 147.762) (width 0.254) (layer "F.Cu") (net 6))
 (segment (start 209.357 147.762) (end 207.899 146.304) (width 0.254) (layer "F.Cu") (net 6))
 (segment (start 251.889599 126.195901) (end 234.306401 126.195901) (width 0.254) (layer "F.Cu") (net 33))
 (segment (start 234.306401 126.195901) (end 233.5355 125.425) (width 0.254) (layer "F.Cu") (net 33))
 (segment (start 252.5605 125.525) (end 251.889599 126.195901) (width 0.254) (layer "F.Cu") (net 33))
 (segment (start 233.5355 120.2515) (end 233.5355 122.125) (width 0.254) (layer "F.Cu") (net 16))
 (segment (start 227.838 118.745) (end 232.029 118.745) (width 0.254) (layer "F.Cu") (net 16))
 (segment (start 232.029 118.745) (end 233.5355 120.2515) (width 0.254) (layer "F.Cu") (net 16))
 (segment (start 251.858349 145.245901) (end 234.456401 145.245901) (width 0.254) (layer "F.Cu") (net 7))
 (segment (start 252.67925 144.425) (end 251.858349 145.245901) (width 0.254) (layer "F.Cu") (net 7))
 (segment (start 234.456401 145.245901) (end 233.6355 144.425) (width 0.254) (layer "F.Cu") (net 7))
 (segment (start 231.974 138.375) (end 233.6355 140.0365) (width 0.254) (layer "F.Cu") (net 12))
 (segment (start 227.798 138.375) (end 231.974 138.375) (width 0.254) (layer "F.Cu") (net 12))
 (segment (start 233.6355 140.0365) (end 233.6355 141.125) (width 0.254) (layer "F.Cu") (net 12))
 (segment (start 246.848 119.325) (end 251.278 119.325) (width 0.254) (layer "F.Cu") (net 4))
 (segment (start 251.278 119.325) (end 252.603 120.65) (width 0.254) (layer "F.Cu") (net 4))
 (segment (start 252.5605 120.6925) (end 252.5605 122.225) (width 0.254) (layer "F.Cu") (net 4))
 (segment (start 252.603 120.65) (end 252.5605 120.6925) (width 0.254) (layer "F.Cu") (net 4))
 (segment (start 251.786 138.375) (end 252.67925 139.26825) (width 0.254) (layer "F.Cu") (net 8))
 (segment (start 246.848 138.375) (end 251.786 138.375) (width 0.254) (layer "F.Cu") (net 8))
 (segment (start 252.67925 139.26825) (end 252.67925 141.125) (width 0.254) (layer "F.Cu") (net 8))
 (segment (start 179 132.137) (end 179 131.5) (width 0.254) (layer "F.Cu") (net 15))
 (segment (start 179 131.5) (end 179 129.75) (width 0.254) (layer "F.Cu") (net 15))
 (segment (start 181.991 135.128) (end 179 132.137) (width 0.254) (layer "F.Cu") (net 15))
 (via (at 179 129.75) (size 0.8) (drill 0.4) (layers "F.Cu" "B.Cu") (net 15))
 (segment (start 180.25 123.25) (end 180.25 123) (width 0.254) (layer "B.Cu") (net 15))
 (segment (start 183.185 121.4565) (end 183.185 120.5815) (width 0.254) (layer "B.Cu") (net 15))
 (segment (start 181.6415 123) (end 183.185 121.4565) (width 0.254) (layer "B.Cu") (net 15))
 (segment (start 179 124.5) (end 180.25 123.25) (width 0.254) (layer "B.Cu") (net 15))
 (segment (start 179 129.75) (end 179 124.5) (width 0.254) (layer "B.Cu") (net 15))
 (segment (start 180.25 123) (end 181.6415 123) (width 0.254) (layer "B.Cu") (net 15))
 (segment (start 221.488 121.285) (end 221.488 137.565) (width 0.254) (layer "B.Cu") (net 11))
 (segment (start 221.488 137.565) (end 222.798 138.875) (width 0.254) (layer "B.Cu") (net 11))
 (segment (start 240.538 121.285) (end 240.538 137.565) (width 0.254) (layer "B.Cu") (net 3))
 (segment (start 240.538 137.565) (end 241.848 138.875) (width 0.254) (layer "B.Cu") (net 3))
 (segment (start 185.585 123.736) (end 186.182 124.333) (width 0.2) (layer "F.Cu") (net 9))
 (segment (start 185.585 120.5815) (end 185.585 123.736) (width 0.2) (layer "F.Cu") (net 9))
 (segment (start 184.785 120.5815) (end 184.785 123.698) (width 0.2) (layer "F.Cu") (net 13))
 (segment (start 184.785 123.698) (end 184.15 124.333) (width 0.2) (layer "F.Cu") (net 13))
 (segment (start 200.633 138.33) (end 200.633 137.311) (width 0.254) (layer "F.Cu") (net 25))
 (segment (start 181.304 143.308) (end 181.356 143.256) (width 0.254) (layer "F.Cu") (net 25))
 (segment (start 181.304 144.708) (end 181.304 143.308) (width 0.254) (layer "F.Cu") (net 25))
 (segment (start 199.263 139.7) (end 200.633 138.33) (width 0.254) (layer "F.Cu") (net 25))
 (segment (start 211.7975 122.101) (end 211.7975 119.7975) (width 0.254) (layer "F.Cu") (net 25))
 (segment (start 181.356 143.256) (end 181.229 143.129) (width 0.254) (layer "F.Cu") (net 25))
 (segment (start 211.7975 119.7975) (end 211.5 119.5) (width 0.254) (layer "F.Cu") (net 25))
 (via (at 199.263 139.7) (size 0.8) (drill 0.4) (layers "F.Cu" "B.Cu") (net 25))
 (via (at 211.5 119.5) (size 0.8) (drill 0.4) (layers "F.Cu" "B.Cu") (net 25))
 (via (at 181.229 143.129) (size 0.8) (drill 0.4) (layers "F.Cu" "B.Cu") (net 25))
 (segment (start 211.5 119.5) (end 194.5 119.5) (width 0.254) (layer "B.Cu") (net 25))
 (segment (start 181.229 143.129) (end 184.658 139.7) (width 0.254) (layer "B.Cu") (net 25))
 (segment (start 194.5 119.5) (end 192.8 121.2) (width 0.254) (layer "B.Cu") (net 25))
 (segment (start 184.658 139.7) (end 192.8 139.7) (width 0.254) (layer "B.Cu") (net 25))
 (segment (start 192.8 139.7) (end 199.136 139.7) (width 0.254) (layer "B.Cu") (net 25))
 (segment (start 192.8 121.2) (end 192.8 139.7) (width 0.254) (layer "B.Cu") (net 25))
 (segment (start 199.136 139.7) (end 199.263 139.7) (width 0.254) (layer "B.Cu") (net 25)))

